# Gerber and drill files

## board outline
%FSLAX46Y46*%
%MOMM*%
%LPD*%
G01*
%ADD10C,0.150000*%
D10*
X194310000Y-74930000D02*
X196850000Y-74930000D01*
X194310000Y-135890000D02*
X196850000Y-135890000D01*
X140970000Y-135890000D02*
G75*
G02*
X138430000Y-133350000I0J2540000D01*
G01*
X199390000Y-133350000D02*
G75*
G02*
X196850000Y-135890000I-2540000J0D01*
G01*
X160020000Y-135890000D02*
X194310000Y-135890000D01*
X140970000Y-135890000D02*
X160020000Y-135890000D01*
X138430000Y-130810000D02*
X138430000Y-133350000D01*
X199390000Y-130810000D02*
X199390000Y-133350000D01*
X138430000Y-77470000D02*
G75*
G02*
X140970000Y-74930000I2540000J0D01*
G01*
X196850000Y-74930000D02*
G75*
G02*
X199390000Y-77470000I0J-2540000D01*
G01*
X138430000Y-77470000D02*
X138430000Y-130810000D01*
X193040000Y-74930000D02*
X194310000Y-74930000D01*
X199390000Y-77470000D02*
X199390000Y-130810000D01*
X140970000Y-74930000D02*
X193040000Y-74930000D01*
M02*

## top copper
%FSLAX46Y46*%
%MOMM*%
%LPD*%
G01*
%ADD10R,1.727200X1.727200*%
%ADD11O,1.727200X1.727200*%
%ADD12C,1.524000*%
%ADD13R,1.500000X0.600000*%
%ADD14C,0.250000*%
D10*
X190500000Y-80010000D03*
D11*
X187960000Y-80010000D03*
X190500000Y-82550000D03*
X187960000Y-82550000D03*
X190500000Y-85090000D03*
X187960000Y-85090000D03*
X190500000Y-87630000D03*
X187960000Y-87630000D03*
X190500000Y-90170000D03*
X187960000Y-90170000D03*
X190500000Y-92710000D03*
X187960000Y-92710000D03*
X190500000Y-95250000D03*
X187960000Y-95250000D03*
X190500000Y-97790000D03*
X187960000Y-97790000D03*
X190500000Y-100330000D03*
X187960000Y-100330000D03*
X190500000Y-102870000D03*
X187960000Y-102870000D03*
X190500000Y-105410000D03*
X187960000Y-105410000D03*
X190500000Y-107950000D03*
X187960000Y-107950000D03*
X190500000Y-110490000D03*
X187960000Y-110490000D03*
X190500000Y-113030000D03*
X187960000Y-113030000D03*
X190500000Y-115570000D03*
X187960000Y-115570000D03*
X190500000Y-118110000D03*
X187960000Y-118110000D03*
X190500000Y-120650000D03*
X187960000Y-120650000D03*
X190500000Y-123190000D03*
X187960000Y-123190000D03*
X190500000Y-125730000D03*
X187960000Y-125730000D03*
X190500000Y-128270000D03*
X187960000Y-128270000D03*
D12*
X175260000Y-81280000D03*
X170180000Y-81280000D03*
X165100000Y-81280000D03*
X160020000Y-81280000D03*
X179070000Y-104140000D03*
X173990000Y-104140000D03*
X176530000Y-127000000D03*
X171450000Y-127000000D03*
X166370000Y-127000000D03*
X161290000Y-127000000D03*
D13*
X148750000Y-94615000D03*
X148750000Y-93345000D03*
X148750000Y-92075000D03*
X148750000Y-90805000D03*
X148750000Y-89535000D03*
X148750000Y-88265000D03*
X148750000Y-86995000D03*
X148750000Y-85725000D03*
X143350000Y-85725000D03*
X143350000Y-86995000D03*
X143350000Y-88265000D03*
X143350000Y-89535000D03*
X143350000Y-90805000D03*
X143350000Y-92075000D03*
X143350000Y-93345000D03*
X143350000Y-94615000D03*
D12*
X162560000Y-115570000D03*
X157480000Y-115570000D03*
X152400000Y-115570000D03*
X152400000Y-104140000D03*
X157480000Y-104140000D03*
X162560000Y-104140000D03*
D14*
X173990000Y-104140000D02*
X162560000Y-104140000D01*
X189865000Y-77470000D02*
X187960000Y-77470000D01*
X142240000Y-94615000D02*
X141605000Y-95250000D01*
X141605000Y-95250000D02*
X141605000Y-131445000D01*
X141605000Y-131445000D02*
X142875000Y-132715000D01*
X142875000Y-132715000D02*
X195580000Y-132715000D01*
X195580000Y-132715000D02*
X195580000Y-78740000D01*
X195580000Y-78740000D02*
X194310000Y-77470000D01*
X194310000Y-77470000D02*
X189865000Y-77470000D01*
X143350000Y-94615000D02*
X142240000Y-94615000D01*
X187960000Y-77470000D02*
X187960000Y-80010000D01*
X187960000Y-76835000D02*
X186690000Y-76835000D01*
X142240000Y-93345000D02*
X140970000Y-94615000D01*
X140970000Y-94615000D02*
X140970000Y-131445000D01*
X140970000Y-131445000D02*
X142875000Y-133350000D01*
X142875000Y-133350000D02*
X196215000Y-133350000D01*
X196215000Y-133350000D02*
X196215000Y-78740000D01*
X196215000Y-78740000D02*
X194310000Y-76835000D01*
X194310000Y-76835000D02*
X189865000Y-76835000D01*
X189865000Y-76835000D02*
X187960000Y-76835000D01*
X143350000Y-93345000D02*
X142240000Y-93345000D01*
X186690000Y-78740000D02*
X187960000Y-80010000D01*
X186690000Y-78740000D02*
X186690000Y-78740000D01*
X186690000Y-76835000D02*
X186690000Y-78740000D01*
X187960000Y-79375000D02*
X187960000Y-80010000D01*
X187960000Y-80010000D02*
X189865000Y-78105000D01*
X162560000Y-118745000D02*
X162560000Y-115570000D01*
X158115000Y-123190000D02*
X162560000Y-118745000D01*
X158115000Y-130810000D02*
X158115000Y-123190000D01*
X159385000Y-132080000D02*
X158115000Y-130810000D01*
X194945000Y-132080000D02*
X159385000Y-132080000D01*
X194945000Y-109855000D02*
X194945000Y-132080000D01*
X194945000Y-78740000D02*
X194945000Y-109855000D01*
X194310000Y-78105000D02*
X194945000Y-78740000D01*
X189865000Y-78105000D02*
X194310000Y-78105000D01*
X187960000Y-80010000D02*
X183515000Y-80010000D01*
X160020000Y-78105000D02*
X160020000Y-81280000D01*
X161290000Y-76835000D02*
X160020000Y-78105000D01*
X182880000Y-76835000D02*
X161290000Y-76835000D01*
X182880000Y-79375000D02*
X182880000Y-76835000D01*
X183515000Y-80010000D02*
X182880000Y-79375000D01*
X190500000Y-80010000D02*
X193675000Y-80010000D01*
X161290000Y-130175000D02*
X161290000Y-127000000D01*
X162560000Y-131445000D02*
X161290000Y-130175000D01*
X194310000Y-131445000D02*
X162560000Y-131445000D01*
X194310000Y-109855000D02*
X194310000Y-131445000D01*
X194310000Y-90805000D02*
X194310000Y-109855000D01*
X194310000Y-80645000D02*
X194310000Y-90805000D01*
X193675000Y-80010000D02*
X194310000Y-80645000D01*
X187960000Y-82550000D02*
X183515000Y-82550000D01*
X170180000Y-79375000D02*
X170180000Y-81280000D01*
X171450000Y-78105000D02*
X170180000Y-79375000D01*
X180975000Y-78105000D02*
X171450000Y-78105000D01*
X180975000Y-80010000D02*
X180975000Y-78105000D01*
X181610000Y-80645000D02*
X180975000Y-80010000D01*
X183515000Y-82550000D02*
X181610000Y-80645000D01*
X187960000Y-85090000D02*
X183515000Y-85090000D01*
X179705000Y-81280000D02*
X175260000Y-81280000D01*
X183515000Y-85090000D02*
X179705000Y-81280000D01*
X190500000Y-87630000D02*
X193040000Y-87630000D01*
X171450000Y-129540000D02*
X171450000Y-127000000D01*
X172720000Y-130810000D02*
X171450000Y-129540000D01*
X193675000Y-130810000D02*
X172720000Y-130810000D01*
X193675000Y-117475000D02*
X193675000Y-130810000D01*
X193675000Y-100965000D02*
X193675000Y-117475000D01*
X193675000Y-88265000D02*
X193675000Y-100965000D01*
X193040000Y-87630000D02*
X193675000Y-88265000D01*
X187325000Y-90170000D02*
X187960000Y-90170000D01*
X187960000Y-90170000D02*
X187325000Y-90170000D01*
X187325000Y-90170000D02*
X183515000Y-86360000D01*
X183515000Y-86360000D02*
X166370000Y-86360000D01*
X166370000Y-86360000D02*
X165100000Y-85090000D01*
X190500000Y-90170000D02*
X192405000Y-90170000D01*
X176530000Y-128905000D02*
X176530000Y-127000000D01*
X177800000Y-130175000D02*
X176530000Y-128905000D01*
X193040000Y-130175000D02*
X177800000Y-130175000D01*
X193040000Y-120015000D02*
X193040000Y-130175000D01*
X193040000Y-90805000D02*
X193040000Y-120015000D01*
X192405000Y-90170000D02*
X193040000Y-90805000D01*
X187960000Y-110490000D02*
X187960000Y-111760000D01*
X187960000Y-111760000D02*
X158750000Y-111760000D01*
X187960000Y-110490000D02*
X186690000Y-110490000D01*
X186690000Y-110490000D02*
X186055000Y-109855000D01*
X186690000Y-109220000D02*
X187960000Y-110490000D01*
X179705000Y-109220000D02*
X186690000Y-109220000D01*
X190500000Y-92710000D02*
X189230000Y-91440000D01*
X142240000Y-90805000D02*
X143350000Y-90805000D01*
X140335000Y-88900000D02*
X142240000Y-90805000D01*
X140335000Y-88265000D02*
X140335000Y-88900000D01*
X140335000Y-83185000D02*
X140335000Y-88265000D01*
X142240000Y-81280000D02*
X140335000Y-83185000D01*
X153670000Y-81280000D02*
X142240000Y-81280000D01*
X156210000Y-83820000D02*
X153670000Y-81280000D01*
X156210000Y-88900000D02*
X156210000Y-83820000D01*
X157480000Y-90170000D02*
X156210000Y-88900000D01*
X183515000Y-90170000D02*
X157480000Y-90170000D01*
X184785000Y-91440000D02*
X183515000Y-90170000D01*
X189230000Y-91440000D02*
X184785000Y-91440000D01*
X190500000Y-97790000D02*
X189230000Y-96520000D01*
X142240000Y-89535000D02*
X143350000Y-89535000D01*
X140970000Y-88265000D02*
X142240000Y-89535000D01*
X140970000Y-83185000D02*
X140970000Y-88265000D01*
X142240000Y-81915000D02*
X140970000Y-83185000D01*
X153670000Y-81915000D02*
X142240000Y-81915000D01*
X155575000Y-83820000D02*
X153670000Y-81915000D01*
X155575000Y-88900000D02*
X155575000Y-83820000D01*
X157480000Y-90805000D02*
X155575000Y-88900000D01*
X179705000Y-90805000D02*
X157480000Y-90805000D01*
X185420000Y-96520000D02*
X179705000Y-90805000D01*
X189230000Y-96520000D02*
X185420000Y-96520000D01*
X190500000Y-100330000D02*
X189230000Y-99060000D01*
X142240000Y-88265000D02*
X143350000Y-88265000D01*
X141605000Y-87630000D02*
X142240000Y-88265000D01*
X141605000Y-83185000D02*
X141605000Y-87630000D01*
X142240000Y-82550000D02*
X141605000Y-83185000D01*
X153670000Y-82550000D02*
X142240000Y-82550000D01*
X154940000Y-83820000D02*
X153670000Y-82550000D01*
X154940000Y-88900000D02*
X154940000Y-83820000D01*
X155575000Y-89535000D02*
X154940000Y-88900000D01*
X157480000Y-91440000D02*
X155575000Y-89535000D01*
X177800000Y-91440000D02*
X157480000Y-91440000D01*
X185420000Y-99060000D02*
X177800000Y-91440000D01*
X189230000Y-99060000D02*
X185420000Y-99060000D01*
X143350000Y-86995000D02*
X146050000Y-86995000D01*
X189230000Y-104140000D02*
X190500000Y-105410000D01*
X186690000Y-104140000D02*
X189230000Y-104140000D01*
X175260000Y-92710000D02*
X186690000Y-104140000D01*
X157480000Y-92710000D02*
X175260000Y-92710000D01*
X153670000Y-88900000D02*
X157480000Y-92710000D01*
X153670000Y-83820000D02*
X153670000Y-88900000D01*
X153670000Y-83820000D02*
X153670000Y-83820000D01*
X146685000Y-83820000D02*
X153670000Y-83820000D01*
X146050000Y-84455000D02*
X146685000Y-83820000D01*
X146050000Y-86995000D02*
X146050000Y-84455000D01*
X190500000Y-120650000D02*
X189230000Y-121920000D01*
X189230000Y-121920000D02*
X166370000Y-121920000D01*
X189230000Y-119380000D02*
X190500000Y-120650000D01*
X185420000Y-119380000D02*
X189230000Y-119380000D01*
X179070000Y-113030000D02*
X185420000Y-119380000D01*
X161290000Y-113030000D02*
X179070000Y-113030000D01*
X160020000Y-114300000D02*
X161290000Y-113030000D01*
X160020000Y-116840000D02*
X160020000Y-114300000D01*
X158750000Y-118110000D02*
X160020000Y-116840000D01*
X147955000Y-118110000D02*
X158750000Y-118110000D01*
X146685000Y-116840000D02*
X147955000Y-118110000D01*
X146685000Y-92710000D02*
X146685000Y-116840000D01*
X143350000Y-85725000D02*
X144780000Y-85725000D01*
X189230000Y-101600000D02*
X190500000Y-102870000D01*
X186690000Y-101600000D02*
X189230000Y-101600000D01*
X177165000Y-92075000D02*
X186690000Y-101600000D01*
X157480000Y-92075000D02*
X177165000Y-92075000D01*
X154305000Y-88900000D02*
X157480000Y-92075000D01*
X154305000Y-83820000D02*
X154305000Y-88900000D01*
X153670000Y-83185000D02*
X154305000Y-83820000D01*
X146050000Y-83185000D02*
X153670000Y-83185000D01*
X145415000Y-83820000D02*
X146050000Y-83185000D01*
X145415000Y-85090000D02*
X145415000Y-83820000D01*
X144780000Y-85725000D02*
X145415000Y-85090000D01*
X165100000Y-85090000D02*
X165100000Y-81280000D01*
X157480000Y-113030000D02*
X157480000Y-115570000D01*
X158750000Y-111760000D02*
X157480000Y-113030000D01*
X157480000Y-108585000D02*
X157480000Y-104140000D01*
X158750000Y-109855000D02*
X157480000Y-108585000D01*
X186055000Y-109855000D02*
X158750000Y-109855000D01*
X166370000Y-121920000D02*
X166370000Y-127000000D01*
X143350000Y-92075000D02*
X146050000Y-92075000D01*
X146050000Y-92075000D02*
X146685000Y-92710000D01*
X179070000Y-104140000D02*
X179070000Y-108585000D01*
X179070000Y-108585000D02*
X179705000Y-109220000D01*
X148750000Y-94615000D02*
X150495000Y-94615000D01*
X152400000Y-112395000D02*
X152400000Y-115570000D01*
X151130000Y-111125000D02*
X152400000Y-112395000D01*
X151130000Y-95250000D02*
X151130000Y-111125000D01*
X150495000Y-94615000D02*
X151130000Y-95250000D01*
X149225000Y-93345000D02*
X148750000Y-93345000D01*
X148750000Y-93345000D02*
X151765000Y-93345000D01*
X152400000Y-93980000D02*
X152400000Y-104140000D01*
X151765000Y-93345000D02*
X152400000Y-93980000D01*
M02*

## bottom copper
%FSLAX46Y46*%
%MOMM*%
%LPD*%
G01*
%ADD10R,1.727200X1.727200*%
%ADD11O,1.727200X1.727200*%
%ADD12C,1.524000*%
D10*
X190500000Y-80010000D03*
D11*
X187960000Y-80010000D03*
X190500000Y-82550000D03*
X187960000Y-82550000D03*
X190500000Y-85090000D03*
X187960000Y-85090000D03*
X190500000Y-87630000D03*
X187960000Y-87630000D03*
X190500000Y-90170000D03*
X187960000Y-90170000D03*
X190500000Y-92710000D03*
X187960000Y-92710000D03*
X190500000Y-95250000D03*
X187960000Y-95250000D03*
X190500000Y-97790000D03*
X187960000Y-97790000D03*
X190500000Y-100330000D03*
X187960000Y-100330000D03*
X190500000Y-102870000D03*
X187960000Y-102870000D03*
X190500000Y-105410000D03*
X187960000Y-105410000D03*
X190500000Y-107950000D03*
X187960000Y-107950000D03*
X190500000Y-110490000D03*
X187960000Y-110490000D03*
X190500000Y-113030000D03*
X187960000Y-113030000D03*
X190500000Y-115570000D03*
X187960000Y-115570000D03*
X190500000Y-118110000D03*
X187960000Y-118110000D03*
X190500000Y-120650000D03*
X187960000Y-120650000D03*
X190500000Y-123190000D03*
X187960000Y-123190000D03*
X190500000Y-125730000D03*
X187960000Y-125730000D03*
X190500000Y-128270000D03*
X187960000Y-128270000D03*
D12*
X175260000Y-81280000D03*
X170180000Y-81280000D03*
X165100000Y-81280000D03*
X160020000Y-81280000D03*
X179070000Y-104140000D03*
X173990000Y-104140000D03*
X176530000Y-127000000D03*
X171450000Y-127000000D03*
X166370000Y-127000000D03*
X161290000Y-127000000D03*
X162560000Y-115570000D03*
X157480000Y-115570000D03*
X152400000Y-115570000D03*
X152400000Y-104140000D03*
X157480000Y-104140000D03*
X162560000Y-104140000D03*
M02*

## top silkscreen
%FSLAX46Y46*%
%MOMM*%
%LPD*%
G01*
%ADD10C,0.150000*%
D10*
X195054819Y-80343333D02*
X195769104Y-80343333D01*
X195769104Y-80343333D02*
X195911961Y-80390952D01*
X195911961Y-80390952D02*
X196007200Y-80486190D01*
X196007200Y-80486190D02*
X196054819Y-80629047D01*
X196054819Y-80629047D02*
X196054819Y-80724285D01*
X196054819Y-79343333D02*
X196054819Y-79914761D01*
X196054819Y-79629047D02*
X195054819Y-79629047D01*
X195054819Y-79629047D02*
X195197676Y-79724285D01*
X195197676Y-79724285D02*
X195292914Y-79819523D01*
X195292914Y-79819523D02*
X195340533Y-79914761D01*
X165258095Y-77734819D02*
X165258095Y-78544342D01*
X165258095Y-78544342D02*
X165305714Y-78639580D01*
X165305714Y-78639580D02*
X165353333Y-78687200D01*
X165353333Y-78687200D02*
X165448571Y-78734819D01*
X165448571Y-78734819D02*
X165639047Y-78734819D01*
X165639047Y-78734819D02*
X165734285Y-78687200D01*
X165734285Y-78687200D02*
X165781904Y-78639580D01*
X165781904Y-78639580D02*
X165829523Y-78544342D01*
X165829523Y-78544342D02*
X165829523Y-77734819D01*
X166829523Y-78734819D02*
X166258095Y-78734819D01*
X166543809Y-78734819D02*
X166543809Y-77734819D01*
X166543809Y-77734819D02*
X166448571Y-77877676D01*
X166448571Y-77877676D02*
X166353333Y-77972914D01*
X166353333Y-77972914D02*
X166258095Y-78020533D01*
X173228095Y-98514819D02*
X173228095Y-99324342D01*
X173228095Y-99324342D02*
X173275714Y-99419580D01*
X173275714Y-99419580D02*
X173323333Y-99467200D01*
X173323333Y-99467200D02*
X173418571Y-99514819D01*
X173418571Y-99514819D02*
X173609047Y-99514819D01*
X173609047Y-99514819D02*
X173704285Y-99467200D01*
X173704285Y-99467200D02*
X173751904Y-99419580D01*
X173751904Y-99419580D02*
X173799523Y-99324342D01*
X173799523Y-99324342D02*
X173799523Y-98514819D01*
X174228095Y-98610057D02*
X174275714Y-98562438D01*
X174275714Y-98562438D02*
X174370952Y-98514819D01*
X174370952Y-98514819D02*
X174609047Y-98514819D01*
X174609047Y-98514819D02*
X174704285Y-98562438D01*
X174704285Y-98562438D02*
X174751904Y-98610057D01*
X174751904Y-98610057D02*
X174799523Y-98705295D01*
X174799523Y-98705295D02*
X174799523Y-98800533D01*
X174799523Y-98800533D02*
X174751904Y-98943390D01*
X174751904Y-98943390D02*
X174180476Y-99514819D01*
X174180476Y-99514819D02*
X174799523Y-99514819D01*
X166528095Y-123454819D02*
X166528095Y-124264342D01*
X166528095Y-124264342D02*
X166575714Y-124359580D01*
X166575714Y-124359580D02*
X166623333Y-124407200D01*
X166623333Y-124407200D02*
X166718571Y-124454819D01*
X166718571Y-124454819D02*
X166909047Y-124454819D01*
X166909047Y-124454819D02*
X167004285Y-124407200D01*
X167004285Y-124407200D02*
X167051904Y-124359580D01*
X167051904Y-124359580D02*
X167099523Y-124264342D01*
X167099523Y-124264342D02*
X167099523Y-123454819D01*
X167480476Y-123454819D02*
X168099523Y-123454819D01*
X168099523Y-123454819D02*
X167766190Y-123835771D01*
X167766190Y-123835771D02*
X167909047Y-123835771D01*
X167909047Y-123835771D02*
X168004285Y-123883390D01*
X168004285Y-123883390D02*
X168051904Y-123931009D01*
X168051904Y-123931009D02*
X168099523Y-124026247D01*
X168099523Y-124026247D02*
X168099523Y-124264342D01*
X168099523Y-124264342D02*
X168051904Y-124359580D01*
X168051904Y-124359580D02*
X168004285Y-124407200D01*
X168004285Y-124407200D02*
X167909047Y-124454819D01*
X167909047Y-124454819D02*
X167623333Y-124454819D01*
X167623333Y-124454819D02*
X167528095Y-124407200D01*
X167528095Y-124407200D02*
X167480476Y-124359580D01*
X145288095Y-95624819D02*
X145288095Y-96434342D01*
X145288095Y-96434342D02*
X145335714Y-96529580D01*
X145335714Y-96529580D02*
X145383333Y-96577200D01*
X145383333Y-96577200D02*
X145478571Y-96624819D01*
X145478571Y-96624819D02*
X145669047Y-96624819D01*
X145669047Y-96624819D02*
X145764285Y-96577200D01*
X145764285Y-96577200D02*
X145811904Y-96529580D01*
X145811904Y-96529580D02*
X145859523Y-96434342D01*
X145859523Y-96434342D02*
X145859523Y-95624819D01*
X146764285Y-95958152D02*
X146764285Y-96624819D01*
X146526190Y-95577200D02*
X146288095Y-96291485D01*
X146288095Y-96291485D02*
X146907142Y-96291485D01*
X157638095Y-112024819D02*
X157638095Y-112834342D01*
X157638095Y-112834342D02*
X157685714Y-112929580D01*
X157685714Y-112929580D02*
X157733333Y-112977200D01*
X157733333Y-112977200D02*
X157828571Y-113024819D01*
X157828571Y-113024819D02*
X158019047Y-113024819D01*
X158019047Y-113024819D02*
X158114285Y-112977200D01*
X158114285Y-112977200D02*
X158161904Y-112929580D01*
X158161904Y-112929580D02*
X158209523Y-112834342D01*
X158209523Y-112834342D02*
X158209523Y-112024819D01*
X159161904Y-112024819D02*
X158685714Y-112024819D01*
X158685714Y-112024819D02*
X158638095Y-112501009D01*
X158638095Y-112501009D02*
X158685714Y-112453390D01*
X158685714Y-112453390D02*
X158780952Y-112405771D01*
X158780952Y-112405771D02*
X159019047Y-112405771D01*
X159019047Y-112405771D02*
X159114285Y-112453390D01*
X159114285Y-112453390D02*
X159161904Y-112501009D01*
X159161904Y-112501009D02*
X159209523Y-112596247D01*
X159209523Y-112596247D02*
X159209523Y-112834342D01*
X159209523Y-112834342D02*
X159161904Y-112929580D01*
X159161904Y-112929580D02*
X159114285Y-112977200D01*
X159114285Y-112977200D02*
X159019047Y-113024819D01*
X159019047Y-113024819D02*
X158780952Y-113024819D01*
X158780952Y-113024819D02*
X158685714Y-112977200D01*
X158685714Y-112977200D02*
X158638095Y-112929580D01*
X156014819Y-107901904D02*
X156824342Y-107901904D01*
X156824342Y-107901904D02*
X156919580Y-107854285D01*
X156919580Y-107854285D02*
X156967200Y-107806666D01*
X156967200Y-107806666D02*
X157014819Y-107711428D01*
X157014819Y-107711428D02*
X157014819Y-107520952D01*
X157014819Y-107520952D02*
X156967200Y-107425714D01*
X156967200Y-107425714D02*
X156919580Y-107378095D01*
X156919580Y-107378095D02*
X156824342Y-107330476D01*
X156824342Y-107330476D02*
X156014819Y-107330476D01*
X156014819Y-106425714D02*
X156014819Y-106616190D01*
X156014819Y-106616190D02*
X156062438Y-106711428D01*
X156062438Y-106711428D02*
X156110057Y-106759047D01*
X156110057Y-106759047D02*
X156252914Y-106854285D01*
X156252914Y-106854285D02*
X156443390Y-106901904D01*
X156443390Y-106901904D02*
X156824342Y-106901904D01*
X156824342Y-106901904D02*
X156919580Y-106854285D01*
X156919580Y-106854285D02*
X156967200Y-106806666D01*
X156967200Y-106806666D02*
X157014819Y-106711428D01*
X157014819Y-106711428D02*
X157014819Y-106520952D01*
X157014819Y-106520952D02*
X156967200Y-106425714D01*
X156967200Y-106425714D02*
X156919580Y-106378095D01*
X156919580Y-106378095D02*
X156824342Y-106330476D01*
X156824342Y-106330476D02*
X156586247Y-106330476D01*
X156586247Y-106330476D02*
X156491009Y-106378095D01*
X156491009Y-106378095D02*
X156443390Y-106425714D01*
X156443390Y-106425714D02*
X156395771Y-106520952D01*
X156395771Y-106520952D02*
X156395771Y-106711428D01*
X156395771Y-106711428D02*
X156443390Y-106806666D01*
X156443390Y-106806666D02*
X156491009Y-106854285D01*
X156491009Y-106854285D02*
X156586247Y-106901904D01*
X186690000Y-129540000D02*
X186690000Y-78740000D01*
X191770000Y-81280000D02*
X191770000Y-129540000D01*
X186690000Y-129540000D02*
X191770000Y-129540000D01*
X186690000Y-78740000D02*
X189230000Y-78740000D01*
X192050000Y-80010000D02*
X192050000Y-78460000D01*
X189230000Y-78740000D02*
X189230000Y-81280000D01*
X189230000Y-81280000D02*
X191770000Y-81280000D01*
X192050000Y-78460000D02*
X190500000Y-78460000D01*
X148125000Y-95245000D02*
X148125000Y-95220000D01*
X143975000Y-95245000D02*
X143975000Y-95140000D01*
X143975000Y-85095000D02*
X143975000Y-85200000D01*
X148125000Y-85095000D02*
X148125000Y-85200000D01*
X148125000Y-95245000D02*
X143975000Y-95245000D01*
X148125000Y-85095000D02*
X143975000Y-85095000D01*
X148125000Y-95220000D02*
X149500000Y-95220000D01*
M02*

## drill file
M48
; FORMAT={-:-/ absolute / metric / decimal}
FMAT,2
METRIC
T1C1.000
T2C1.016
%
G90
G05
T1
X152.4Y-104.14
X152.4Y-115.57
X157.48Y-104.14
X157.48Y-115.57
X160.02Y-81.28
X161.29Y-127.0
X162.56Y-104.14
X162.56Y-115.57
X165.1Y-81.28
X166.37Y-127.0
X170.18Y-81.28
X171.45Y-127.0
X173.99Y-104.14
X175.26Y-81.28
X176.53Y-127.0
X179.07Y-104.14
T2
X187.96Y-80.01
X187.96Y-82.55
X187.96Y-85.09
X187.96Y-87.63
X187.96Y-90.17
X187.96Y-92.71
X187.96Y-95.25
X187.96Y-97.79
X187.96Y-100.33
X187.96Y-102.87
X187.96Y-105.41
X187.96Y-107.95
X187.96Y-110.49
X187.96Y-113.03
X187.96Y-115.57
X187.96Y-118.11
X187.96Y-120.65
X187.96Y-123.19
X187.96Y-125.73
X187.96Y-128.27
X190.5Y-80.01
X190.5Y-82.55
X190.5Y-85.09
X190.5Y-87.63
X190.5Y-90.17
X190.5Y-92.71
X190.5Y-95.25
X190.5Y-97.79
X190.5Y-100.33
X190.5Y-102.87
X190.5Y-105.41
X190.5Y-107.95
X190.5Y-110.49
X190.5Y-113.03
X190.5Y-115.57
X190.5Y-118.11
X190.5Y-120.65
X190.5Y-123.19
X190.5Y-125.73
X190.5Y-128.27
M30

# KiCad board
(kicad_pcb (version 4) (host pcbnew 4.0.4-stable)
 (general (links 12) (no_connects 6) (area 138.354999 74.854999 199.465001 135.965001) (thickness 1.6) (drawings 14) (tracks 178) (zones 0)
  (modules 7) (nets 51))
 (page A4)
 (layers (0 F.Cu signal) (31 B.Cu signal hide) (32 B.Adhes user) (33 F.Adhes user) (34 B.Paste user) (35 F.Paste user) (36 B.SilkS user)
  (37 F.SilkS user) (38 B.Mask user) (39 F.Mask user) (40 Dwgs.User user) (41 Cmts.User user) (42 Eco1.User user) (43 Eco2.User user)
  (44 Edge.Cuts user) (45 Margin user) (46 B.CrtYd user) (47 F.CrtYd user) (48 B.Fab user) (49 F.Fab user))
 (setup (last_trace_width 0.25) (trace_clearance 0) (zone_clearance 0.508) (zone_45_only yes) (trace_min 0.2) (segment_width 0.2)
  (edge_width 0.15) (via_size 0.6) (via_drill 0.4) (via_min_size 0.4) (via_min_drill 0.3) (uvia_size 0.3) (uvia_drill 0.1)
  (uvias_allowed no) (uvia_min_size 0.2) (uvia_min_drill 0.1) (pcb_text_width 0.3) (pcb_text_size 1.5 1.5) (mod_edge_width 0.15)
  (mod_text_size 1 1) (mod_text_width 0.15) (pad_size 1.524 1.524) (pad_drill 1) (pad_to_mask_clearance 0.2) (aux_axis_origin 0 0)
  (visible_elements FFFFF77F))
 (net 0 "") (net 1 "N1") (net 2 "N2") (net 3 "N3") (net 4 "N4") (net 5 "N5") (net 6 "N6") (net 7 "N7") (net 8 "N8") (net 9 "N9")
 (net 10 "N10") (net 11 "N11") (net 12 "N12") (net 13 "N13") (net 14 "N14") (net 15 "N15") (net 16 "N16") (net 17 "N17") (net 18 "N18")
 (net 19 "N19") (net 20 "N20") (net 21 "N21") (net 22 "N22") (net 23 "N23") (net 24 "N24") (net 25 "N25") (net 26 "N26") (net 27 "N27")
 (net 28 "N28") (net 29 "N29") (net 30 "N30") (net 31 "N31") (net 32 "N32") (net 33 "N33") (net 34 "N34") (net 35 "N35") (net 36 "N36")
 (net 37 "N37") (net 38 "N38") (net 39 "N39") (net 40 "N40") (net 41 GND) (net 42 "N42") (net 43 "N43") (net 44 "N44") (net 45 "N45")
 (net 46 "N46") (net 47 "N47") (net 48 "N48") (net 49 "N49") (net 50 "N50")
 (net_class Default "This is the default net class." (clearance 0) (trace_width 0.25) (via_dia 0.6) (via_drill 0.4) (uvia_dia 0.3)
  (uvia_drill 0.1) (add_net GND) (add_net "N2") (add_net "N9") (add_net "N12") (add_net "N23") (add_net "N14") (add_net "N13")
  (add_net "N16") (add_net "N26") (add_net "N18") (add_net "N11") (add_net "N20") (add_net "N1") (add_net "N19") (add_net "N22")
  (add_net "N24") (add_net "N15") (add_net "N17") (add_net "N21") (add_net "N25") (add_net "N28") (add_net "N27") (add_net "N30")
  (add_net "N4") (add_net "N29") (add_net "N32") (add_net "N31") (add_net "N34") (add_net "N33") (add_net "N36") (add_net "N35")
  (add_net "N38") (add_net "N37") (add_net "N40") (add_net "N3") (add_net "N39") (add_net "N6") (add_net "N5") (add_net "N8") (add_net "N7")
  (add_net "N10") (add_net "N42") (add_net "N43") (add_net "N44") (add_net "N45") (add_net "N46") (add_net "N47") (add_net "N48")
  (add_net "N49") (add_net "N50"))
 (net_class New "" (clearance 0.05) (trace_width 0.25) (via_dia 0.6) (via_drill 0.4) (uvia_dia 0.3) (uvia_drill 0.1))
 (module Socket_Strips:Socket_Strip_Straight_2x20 (layer F.Cu) (at 190.5 80.01 270)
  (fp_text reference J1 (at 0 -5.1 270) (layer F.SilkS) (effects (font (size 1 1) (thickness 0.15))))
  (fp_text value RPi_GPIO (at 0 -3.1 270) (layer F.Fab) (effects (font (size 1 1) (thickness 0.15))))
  (fp_line (start 49.53 3.81) (end -1.27 3.81) (layer F.SilkS) (width 0.15))
  (fp_line (start 1.27 -1.27) (end 49.53 -1.27) (layer F.SilkS) (width 0.15))
  (fp_line (start 49.53 3.81) (end 49.53 -1.27) (layer F.SilkS) (width 0.15))
  (fp_line (start -1.27 3.81) (end -1.27 1.27) (layer F.SilkS) (width 0.15))
  (fp_line (start 0 -1.55) (end -1.55 -1.55) (layer F.SilkS) (width 0.15))
  (fp_line (start -1.27 1.27) (end 1.27 1.27) (layer F.SilkS) (width 0.15))
  (fp_line (start 1.27 1.27) (end 1.27 -1.27) (layer F.SilkS) (width 0.15))
  (fp_line (start -1.55 -1.55) (end -1.55 0) (layer F.SilkS) (width 0.15))
  (pad 2 thru_hole rect (at 0 0 270) (size 1.7272 1.7272) (drill 1.016) (layers *.Cu *.Mask) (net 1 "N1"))
  (pad 1 thru_hole oval (at 0 2.54 270) (size 1.7272 1.7272) (drill 1.016) (layers *.Cu *.Mask) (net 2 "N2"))
  (pad 4 thru_hole oval (at 2.54 0 270) (size 1.7272 1.7272) (drill 1.016) (layers *.Cu *.Mask) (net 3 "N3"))
  (pad 3 thru_hole oval (at 2.54 2.54 270) (size 1.7272 1.7272) (drill 1.016) (layers *.Cu *.Mask) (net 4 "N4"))
  (pad 6 thru_hole oval (at 5.08 0 270) (size 1.7272 1.7272) (drill 1.016) (layers *.Cu *.Mask) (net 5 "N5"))
  (pad 5 thru_hole oval (at 5.08 2.54 270) (size 1.7272 1.7272) (drill 1.016) (layers *.Cu *.Mask) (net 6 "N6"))
  (pad 8 thru_hole oval (at 7.62 0 270) (size 1.7272 1.7272) (drill 1.016) (layers *.Cu *.Mask) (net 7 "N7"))
  (pad 7 thru_hole oval (at 7.62 2.54 270) (size 1.7272 1.7272) (drill 1.016) (layers *.Cu *.Mask) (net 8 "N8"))
  (pad 10 thru_hole oval (at 10.16 0 270) (size 1.7272 1.7272) (drill 1.016) (layers *.Cu *.Mask) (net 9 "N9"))
  (pad 9 thru_hole oval (at 10.16 2.54 270) (size 1.7272 1.7272) (drill 1.016) (layers *.Cu *.Mask) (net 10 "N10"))
  (pad 18 thru_hole oval (at 12.7 0 270) (size 1.7272 1.7272) (drill 1.016) (layers *.Cu *.Mask) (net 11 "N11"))
  (pad 11 thru_hole oval (at 12.7 2.54 270) (size 1.7272 1.7272) (drill 1.016) (layers *.Cu *.Mask) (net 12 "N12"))
  (pad 14 thru_hole oval (at 15.24 0 270) (size 1.7272 1.7272) (drill 1.016) (layers *.Cu *.Mask) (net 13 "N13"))
  (pad 13 thru_hole oval (at 15.24 2.54 270) (size 1.7272 1.7272) (drill 1.016) (layers *.Cu *.Mask) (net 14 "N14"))
  (pad 23 thru_hole oval (at 17.78 0 270) (size 1.7272 1.7272) (drill 1.016) (layers *.Cu *.Mask) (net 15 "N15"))
  (pad 15 thru_hole oval (at 17.78 2.54 270) (size 1.7272 1.7272) (drill 1.016) (layers *.Cu *.Mask) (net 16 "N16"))
  (pad 24 thru_hole oval (at 20.32 0 270) (size 1.7272 1.7272) (drill 1.016) (layers *.Cu *.Mask) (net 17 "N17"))
  (pad 17 thru_hole oval (at 20.32 2.54 270) (size 1.7272 1.7272) (drill 1.016) (layers *.Cu *.Mask) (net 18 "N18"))
  (pad 20 thru_hole oval (at 22.86 0 270) (size 1.7272 1.7272) (drill 1.016) (layers *.Cu *.Mask) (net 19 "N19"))
  (pad 19 thru_hole oval (at 22.86 2.54 270) (size 1.7272 1.7272) (drill 1.016) (layers *.Cu *.Mask) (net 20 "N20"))
  (pad 25 thru_hole oval (at 25.4 0 270) (size 1.7272 1.7272) (drill 1.016) (layers *.Cu *.Mask) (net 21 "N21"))
  (pad 21 thru_hole oval (at 25.4 2.54 270) (size 1.7272 1.7272) (drill 1.016) (layers *.Cu *.Mask) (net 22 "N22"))
  (pad 12 thru_hole oval (at 27.94 0 270) (size 1.7272 1.7272) (drill 1.016) (layers *.Cu *.Mask) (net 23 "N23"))
  (pad 22 thru_hole oval (at 27.94 2.54 270) (size 1.7272 1.7272) (drill 1.016) (layers *.Cu *.Mask) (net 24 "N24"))
  (pad 26 thru_hole oval (at 30.48 0 270) (size 1.7272 1.7272) (drill 1.016) (layers *.Cu *.Mask) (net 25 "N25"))
  (pad 16 thru_hole oval (at 30.48 2.54 270) (size 1.7272 1.7272) (drill 1.016) (layers *.Cu *.Mask) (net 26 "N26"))
  (pad 28 thru_hole oval (at 33.02 0 270) (size 1.7272 1.7272) (drill 1.016) (layers *.Cu *.Mask) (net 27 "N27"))
  (pad 27 thru_hole oval (at 33.02 2.54 270) (size 1.7272 1.7272) (drill 1.016) (layers *.Cu *.Mask) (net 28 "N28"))
  (pad 30 thru_hole oval (at 35.56 0 270) (size 1.7272 1.7272) (drill 1.016) (layers *.Cu *.Mask) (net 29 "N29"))
  (pad 29 thru_hole oval (at 35.56 2.54 270) (size 1.7272 1.7272) (drill 1.016) (layers *.Cu *.Mask) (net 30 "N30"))
  (pad 32 thru_hole oval (at 38.1 0 270) (size 1.7272 1.7272) (drill 1.016) (layers *.Cu *.Mask) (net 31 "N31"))
  (pad 31 thru_hole oval (at 38.1 2.54 270) (size 1.7272 1.7272) (drill 1.016) (layers *.Cu *.Mask) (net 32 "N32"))
  (pad 34 thru_hole oval (at 40.64 0 270) (size 1.7272 1.7272) (drill 1.016) (layers *.Cu *.Mask) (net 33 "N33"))
  (pad 33 thru_hole oval (at 40.64 2.54 270) (size 1.7272 1.7272) (drill 1.016) (layers *.Cu *.Mask) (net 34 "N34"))
  (pad 36 thru_hole oval (at 43.18 0 270) (size 1.7272 1.7272) (drill 1.016) (layers *.Cu *.Mask) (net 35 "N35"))
  (pad 35 thru_hole oval (at 43.18 2.54 270) (size 1.7272 1.7272) (drill 1.016) (layers *.Cu *.Mask) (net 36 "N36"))
  (pad 38 thru_hole oval (at 45.72 0 270) (size 1.7272 1.7272) (drill 1.016) (layers *.Cu *.Mask) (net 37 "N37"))
  (pad 37 thru_hole oval (at 45.72 2.54 270) (size 1.7272 1.7272) (drill 1.016) (layers *.Cu *.Mask) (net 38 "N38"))
  (pad 40 thru_hole oval (at 48.26 0 270) (size 1.7272 1.7272) (drill 1.016) (layers *.Cu *.Mask) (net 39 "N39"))
  (pad 39 thru_hole oval (at 48.26 2.54 270) (size 1.7272 1.7272) (drill 1.016) (layers *.Cu *.Mask) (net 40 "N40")))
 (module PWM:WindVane (layer F.Cu) (at 160.02 81.28)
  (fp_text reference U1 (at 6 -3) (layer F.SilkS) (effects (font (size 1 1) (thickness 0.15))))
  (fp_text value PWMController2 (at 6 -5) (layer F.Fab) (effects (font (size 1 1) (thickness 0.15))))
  (pad 4 thru_hole circle (at 15.24 0) (size 1.524 1.524) (drill 1) (layers *.Cu *.Mask))
  (pad 3 thru_hole circle (at 10.16 0) (size 1.524 1.524) (drill 1) (layers *.Cu *.Mask))
  (pad 2 thru_hole circle (at 5.08 0) (size 1.524 1.524) (drill 1) (layers *.Cu *.Mask) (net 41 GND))
  (pad 1 thru_hole circle (at 0 0) (size 1.524 1.524) (drill 1) (layers *.Cu *.Mask)))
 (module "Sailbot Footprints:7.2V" (layer F.Cu) (at 173.99 104.14)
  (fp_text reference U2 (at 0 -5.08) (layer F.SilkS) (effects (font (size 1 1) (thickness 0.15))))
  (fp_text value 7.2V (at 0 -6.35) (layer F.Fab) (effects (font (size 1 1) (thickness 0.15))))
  (pad 2 thru_hole circle (at 5.08 0) (size 1.524 1.524) (drill 1) (layers *.Cu *.Mask) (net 41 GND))
  (pad 1 thru_hole circle (at 0 0) (size 1.524 1.524) (drill 1) (layers *.Cu *.Mask) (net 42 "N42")))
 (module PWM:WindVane (layer F.Cu) (at 161.29 127)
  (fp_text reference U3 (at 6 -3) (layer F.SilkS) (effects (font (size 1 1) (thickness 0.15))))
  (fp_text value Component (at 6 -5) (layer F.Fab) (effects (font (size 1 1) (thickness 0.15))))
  (pad 4 thru_hole circle (at 15.24 0) (size 1.524 1.524) (drill 1) (layers *.Cu *.Mask))
  (pad 3 thru_hole circle (at 10.16 0) (size 1.524 1.524) (drill 1) (layers *.Cu *.Mask))
  (pad 2 thru_hole circle (at 5.08 0) (size 1.524 1.524) (drill 1) (layers *.Cu *.Mask) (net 41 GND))
  (pad 1 thru_hole circle (at 0 0) (size 1.524 1.524) (drill 1) (layers *.Cu *.Mask)))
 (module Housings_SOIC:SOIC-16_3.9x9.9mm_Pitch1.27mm (layer F.Cu) (at 146.05 90.17 180)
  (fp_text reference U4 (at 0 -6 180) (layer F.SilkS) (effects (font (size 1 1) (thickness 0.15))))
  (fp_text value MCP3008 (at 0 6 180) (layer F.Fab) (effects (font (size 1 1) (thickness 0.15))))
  (fp_line (start -2.075 -5.075) (end -2.075 -5.05) (layer F.SilkS) (width 0.15))
  (fp_line (start 2.075 -5.075) (end 2.075 -4.97) (layer F.SilkS) (width 0.15))
  (fp_line (start 2.075 5.075) (end 2.075 4.97) (layer F.SilkS) (width 0.15))
  (fp_line (start -2.075 5.075) (end -2.075 4.97) (layer F.SilkS) (width 0.15))
  (fp_line (start -2.075 -5.075) (end 2.075 -5.075) (layer F.SilkS) (width 0.15))
  (fp_line (start -2.075 5.075) (end 2.075 5.075) (layer F.SilkS) (width 0.15))
  (fp_line (start -2.075 -5.05) (end -3.45 -5.05) (layer F.SilkS) (width 0.15))
  (pad 1 smd rect (at -2.7 -4.445 180) (size 1.5 0.6) (layers F.Cu F.Paste F.Mask) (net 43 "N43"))
  (pad 2 smd rect (at -2.7 -3.175 180) (size 1.5 0.6) (layers F.Cu F.Paste F.Mask) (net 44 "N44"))
  (pad 3 smd rect (at -2.7 -1.905 180) (size 1.5 0.6) (layers F.Cu F.Paste F.Mask) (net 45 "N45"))
  (pad 4 smd rect (at -2.7 -0.635 180) (size 1.5 0.6) (layers F.Cu F.Paste F.Mask) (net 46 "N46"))
  (pad 5 smd rect (at -2.7 0.635 180) (size 1.5 0.6) (layers F.Cu F.Paste F.Mask) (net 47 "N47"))
  (pad 6 smd rect (at -2.7 1.905 180) (size 1.5 0.6) (layers F.Cu F.Paste F.Mask) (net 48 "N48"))
  (pad 7 smd rect (at -2.7 3.175 180) (size 1.5 0.6) (layers F.Cu F.Paste F.Mask) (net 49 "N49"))
  (pad 8 smd rect (at -2.7 4.445 180) (size 1.5 0.6) (layers F.Cu F.Paste F.Mask) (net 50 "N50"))
  (pad 9 smd rect (at 2.7 4.445 180) (size 1.5 0.6) (layers F.Cu F.Paste F.Mask) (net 41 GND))
  (pad 10 smd rect (at 2.7 3.175 180) (size 1.5 0.6) (layers F.Cu F.Paste F.Mask) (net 21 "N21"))
  (pad 11 smd rect (at 2.7 1.905 180) (size 1.5 0.6) (layers F.Cu F.Paste F.Mask) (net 17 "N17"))
  (pad 12 smd rect (at 2.7 0.635 180) (size 1.5 0.6) (layers F.Cu F.Paste F.Mask) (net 15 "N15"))
  (pad 13 smd rect (at 2.7 -0.635 180) (size 1.5 0.6) (layers F.Cu F.Paste F.Mask) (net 11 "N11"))
  (pad 14 smd rect (at 2.7 -1.905 180) (size 1.5 0.6) (layers F.Cu F.Paste F.Mask) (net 41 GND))
  (pad 15 smd rect (at 2.7 -3.175 180) (size 1.5 0.6) (layers F.Cu F.Paste F.Mask) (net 2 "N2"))
  (pad 16 smd rect (at 2.7 -4.445 180) (size 1.5 0.6) (layers F.Cu F.Paste F.Mask) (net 2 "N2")))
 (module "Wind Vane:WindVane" (layer F.Cu) (at 152.4 115.57)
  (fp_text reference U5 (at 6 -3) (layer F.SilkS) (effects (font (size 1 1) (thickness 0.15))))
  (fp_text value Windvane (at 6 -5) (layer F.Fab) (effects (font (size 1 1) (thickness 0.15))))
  (pad 3 thru_hole circle (at 10.16 0) (size 1.524 1.524) (drill 1) (layers *.Cu *.Mask))
  (pad 2 thru_hole circle (at 5.08 0) (size 1.524 1.524) (drill 1) (layers *.Cu *.Mask) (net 41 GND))
  (pad 1 thru_hole circle (at 0 0) (size 1.524 1.524) (drill 1) (layers *.Cu *.Mask)))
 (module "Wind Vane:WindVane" (layer F.Cu) (at 162.56 104.14 180)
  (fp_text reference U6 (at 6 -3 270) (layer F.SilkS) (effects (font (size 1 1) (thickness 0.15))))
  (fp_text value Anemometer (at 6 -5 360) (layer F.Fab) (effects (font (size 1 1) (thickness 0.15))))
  (pad 3 thru_hole circle (at 10.16 0 180) (size 1.524 1.524) (drill 1) (layers *.Cu *.Mask))
  (pad 2 thru_hole circle (at 5.08 0 180) (size 1.524 1.524) (drill 1) (layers *.Cu *.Mask) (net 41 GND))
  (pad 1 thru_hole circle (at 0 0 180) (size 1.524 1.524) (drill 1) (layers *.Cu *.Mask)))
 (gr_line (start 194.31 74.93) (end 196.85 74.93) (angle 90) (layer Edge.Cuts) (width 0.15))
 (gr_line (start 194.31 135.89) (end 196.85 135.89) (angle 90) (layer Edge.Cuts) (width 0.15))
 (gr_arc (start 140.97 133.35) (end 140.97 135.89) (angle 90) (layer Edge.Cuts) (width 0.15))
 (gr_arc (start 196.85 133.35) (end 199.39 133.35) (angle 90) (layer Edge.Cuts) (width 0.15))
 (gr_line (start 160.02 135.89) (end 194.31 135.89) (angle 90) (layer Edge.Cuts) (width 0.15))
 (gr_line (start 140.97 135.89) (end 160.02 135.89) (angle 90) (layer Edge.Cuts) (width 0.15))
 (gr_line (start 138.43 130.81) (end 138.43 133.35) (angle 90) (layer Edge.Cuts) (width 0.15))
 (gr_line (start 199.39 130.81) (end 199.39 133.35) (angle 90) (layer Edge.Cuts) (width 0.15))
 (gr_arc (start 140.97 77.47) (end 138.43 77.47) (angle 90) (layer Edge.Cuts) (width 0.15))
 (gr_arc (start 196.85 77.47) (end 196.85 74.93) (angle 90) (layer Edge.Cuts) (width 0.15))
 (gr_line (start 138.43 77.47) (end 138.43 130.81) (angle 90) (layer Edge.Cuts) (width 0.15))
 (gr_line (start 193.04 74.93) (end 194.31 74.93) (angle 90) (layer Edge.Cuts) (width 0.15))
 (gr_line (start 199.39 77.47) (end 199.39 130.81) (angle 90) (layer Edge.Cuts) (width 0.15))
 (gr_line (start 140.97 74.93) (end 193.04 74.93) (angle 90) (layer Edge.Cuts) (width 0.15))
 (segment (start 173.99 104.14) (end 162.56 104.14) (width 0.25) (layer F.Cu) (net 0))
 (segment (start 189.865 77.47) (end 187.96 77.47) (width 0.25) (layer F.Cu) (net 2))
 (segment (start 142.24 94.615) (end 141.605 95.25) (width 0.25) (layer F.Cu) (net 2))
 (segment (start 141.605 95.25) (end 141.605 131.445) (width 0.25) (layer F.Cu) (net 2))
 (segment (start 141.605 131.445) (end 142.875 132.715) (width 0.25) (layer F.Cu) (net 2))
 (segment (start 142.875 132.715) (end 195.58 132.715) (width 0.25) (layer F.Cu) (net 2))
 (segment (start 195.58 132.715) (end 195.58 78.74) (width 0.25) (layer F.Cu) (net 2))
 (segment (start 195.58 78.74) (end 194.31 77.47) (width 0.25) (layer F.Cu) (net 2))
 (segment (start 194.31 77.47) (end 189.865 77.47) (width 0.25) (layer F.Cu) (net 2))
 (segment (start 143.35 94.615) (end 142.24 94.615) (width 0.25) (layer F.Cu) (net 2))
 (segment (start 187.96 77.47) (end 187.96 80.01) (width 0.25) (layer F.Cu) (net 2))
 (segment (start 187.96 76.835) (end 186.69 76.835) (width 0.25) (layer F.Cu) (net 2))
 (segment (start 142.24 93.345) (end 140.97 94.615) (width 0.25) (layer F.Cu) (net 2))
 (segment (start 140.97 94.615) (end 140.97 131.445) (width 0.25) (layer F.Cu) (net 2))
 (segment (start 140.97 131.445) (end 142.875 133.35) (width 0.25) (layer F.Cu) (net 2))
 (segment (start 142.875 133.35) (end 196.215 133.35) (width 0.25) (layer F.Cu) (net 2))
 (segment (start 196.215 133.35) (end 196.215 78.74) (width 0.25) (layer F.Cu) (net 2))
 (segment (start 196.215 78.74) (end 194.31 76.835) (width 0.25) (layer F.Cu) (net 2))
 (segment (start 194.31 76.835) (end 189.865 76.835) (width 0.25) (layer F.Cu) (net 2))
 (segment (start 189.865 76.835) (end 187.96 76.835) (width 0.25) (layer F.Cu) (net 2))
 (segment (start 143.35 93.345) (end 142.24 93.345) (width 0.25) (layer F.Cu) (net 2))
 (segment (start 186.69 78.74) (end 187.96 80.01) (width 0.25) (layer F.Cu) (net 2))
 (segment (start 186.69 78.74) (end 186.69 78.74) (width 0.25) (layer F.Cu) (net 2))
 (segment (start 186.69 76.835) (end 186.69 78.74) (width 0.25) (layer F.Cu) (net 2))
 (segment (start 187.96 79.375) (end 187.96 80.01) (width 0.25) (layer F.Cu) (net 2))
 (segment (start 187.96 80.01) (end 189.865 78.105) (width 0.25) (layer F.Cu) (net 2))
 (segment (start 162.56 118.745) (end 162.56 115.57) (width 0.25) (layer F.Cu) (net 2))
 (segment (start 158.115 123.19) (end 162.56 118.745) (width 0.25) (layer F.Cu) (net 2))
 (segment (start 158.115 130.81) (end 158.115 123.19) (width 0.25) (layer F.Cu) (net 2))
 (segment (start 159.385 132.08) (end 158.115 130.81) (width 0.25) (layer F.Cu) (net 2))
 (segment (start 194.945 132.08) (end 159.385 132.08) (width 0.25) (layer F.Cu) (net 2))
 (segment (start 194.945 109.855) (end 194.945 132.08) (width 0.25) (layer F.Cu) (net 2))
 (segment (start 194.945 78.74) (end 194.945 109.855) (width 0.25) (layer F.Cu) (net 2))
 (segment (start 194.31 78.105) (end 194.945 78.74) (width 0.25) (layer F.Cu) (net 2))
 (segment (start 189.865 78.105) (end 194.31 78.105) (width 0.25) (layer F.Cu) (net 2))
 (segment (start 187.96 80.01) (end 183.515 80.01) (width 0.25) (layer F.Cu) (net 2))
 (segment (start 160.02 78.105) (end 160.02 81.28) (width 0.25) (layer F.Cu) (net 2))
 (segment (start 161.29 76.835) (end 160.02 78.105) (width 0.25) (layer F.Cu) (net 2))
 (segment (start 182.88 76.835) (end 161.29 76.835) (width 0.25) (layer F.Cu) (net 2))
 (segment (start 182.88 79.375) (end 182.88 76.835) (width 0.25) (layer F.Cu) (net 2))
 (segment (start 183.515 80.01) (end 182.88 79.375) (width 0.25) (layer F.Cu) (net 2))
 (segment (start 190.5 80.01) (end 193.675 80.01) (width 0.25) (layer F.Cu) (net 1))
 (segment (start 161.29 130.175) (end 161.29 127) (width 0.25) (layer F.Cu) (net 1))
 (segment (start 162.56 131.445) (end 161.29 130.175) (width 0.25) (layer F.Cu) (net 1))
 (segment (start 194.31 131.445) (end 162.56 131.445) (width 0.25) (layer F.Cu) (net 1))
 (segment (start 194.31 109.855) (end 194.31 131.445) (width 0.25) (layer F.Cu) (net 1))
 (segment (start 194.31 90.805) (end 194.31 109.855) (width 0.25) (layer F.Cu) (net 1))
 (segment (start 194.31 80.645) (end 194.31 90.805) (width 0.25) (layer F.Cu) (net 1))
 (segment (start 193.675 80.01) (end 194.31 80.645) (width 0.25) (layer F.Cu) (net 1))
 (segment (start 187.96 82.55) (end 183.515 82.55) (width 0.25) (layer F.Cu) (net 4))
 (segment (start 170.18 79.375) (end 170.18 81.28) (width 0.25) (layer F.Cu) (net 4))
 (segment (start 171.45 78.105) (end 170.18 79.375) (width 0.25) (layer F.Cu) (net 4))
 (segment (start 180.975 78.105) (end 171.45 78.105) (width 0.25) (layer F.Cu) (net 4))
 (segment (start 180.975 80.01) (end 180.975 78.105) (width 0.25) (layer F.Cu) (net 4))
 (segment (start 181.61 80.645) (end 180.975 80.01) (width 0.25) (layer F.Cu) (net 4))
 (segment (start 183.515 82.55) (end 181.61 80.645) (width 0.25) (layer F.Cu) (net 4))
 (segment (start 187.96 85.09) (end 183.515 85.09) (width 0.25) (layer F.Cu) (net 6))
 (segment (start 179.705 81.28) (end 175.26 81.28) (width 0.25) (layer F.Cu) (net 6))
 (segment (start 183.515 85.09) (end 179.705 81.28) (width 0.25) (layer F.Cu) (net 6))
 (segment (start 190.5 87.63) (end 193.04 87.63) (width 0.25) (layer F.Cu) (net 7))
 (segment (start 171.45 129.54) (end 171.45 127) (width 0.25) (layer F.Cu) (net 7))
 (segment (start 172.72 130.81) (end 171.45 129.54) (width 0.25) (layer F.Cu) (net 7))
 (segment (start 193.675 130.81) (end 172.72 130.81) (width 0.25) (layer F.Cu) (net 7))
 (segment (start 193.675 117.475) (end 193.675 130.81) (width 0.25) (layer F.Cu) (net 7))
 (segment (start 193.675 100.965) (end 193.675 117.475) (width 0.25) (layer F.Cu) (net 7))
 (segment (start 193.675 88.265) (end 193.675 100.965) (width 0.25) (layer F.Cu) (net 7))
 (segment (start 193.04 87.63) (end 193.675 88.265) (width 0.25) (layer F.Cu) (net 7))
 (segment (start 187.325 90.17) (end 187.96 90.17) (width 0.25) (layer F.Cu) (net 10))
 (segment (start 187.96 90.17) (end 187.325 90.17) (width 0.25) (layer F.Cu) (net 10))
 (segment (start 187.325 90.17) (end 183.515 86.36) (width 0.25) (layer F.Cu) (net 10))
 (segment (start 183.515 86.36) (end 166.37 86.36) (width 0.25) (layer F.Cu) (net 10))
 (segment (start 166.37 86.36) (end 165.1 85.09) (width 0.25) (layer F.Cu) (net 10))
 (segment (start 190.5 90.17) (end 192.405 90.17) (width 0.25) (layer F.Cu) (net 9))
 (segment (start 176.53 128.905) (end 176.53 127) (width 0.25) (layer F.Cu) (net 9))
 (segment (start 177.8 130.175) (end 176.53 128.905) (width 0.25) (layer F.Cu) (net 9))
 (segment (start 193.04 130.175) (end 177.8 130.175) (width 0.25) (layer F.Cu) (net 9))
 (segment (start 193.04 120.015) (end 193.04 130.175) (width 0.25) (layer F.Cu) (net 9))
 (segment (start 193.04 90.805) (end 193.04 120.015) (width 0.25) (layer F.Cu) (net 9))
 (segment (start 192.405 90.17) (end 193.04 90.805) (width 0.25) (layer F.Cu) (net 9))
 (segment (start 187.96 110.49) (end 187.96 111.76) (width 0.25) (layer F.Cu) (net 26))
 (segment (start 187.96 111.76) (end 158.75 111.76) (width 0.25) (layer F.Cu) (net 26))
 (segment (start 187.96 110.49) (end 186.69 110.49) (width 0.25) (layer F.Cu) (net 26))
 (segment (start 186.69 110.49) (end 186.055 109.855) (width 0.25) (layer F.Cu) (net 26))
 (segment (start 186.69 109.22) (end 187.96 110.49) (width 0.25) (layer F.Cu) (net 26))
 (segment (start 179.705 109.22) (end 186.69 109.22) (width 0.25) (layer F.Cu) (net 26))
 (segment (start 190.5 92.71) (end 189.23 91.44) (width 0.25) (layer F.Cu) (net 11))
 (segment (start 142.24 90.805) (end 143.35 90.805) (width 0.25) (layer F.Cu) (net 11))
 (segment (start 140.335 88.9) (end 142.24 90.805) (width 0.25) (layer F.Cu) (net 11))
 (segment (start 140.335 88.265) (end 140.335 88.9) (width 0.25) (layer F.Cu) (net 11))
 (segment (start 140.335 83.185) (end 140.335 88.265) (width 0.25) (layer F.Cu) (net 11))
 (segment (start 142.24 81.28) (end 140.335 83.185) (width 0.25) (layer F.Cu) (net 11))
 (segment (start 153.67 81.28) (end 142.24 81.28) (width 0.25) (layer F.Cu) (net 11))
 (segment (start 156.21 83.82) (end 153.67 81.28) (width 0.25) (layer F.Cu) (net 11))
 (segment (start 156.21 88.9) (end 156.21 83.82) (width 0.25) (layer F.Cu) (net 11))
 (segment (start 157.48 90.17) (end 156.21 88.9) (width 0.25) (layer F.Cu) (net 11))
 (segment (start 183.515 90.17) (end 157.48 90.17) (width 0.25) (layer F.Cu) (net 11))
 (segment (start 184.785 91.44) (end 183.515 90.17) (width 0.25) (layer F.Cu) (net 11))
 (segment (start 189.23 91.44) (end 184.785 91.44) (width 0.25) (layer F.Cu) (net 11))
 (segment (start 190.5 97.79) (end 189.23 96.52) (width 0.25) (layer F.Cu) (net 15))
 (segment (start 142.24 89.535) (end 143.35 89.535) (width 0.25) (layer F.Cu) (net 15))
 (segment (start 140.97 88.265) (end 142.24 89.535) (width 0.25) (layer F.Cu) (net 15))
 (segment (start 140.97 83.185) (end 140.97 88.265) (width 0.25) (layer F.Cu) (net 15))
 (segment (start 142.24 81.915) (end 140.97 83.185) (width 0.25) (layer F.Cu) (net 15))
 (segment (start 153.67 81.915) (end 142.24 81.915) (width 0.25) (layer F.Cu) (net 15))
 (segment (start 155.575 83.82) (end 153.67 81.915) (width 0.25) (layer F.Cu) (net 15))
 (segment (start 155.575 88.9) (end 155.575 83.82) (width 0.25) (layer F.Cu) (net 15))
 (segment (start 157.48 90.805) (end 155.575 88.9) (width 0.25) (layer F.Cu) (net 15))
 (segment (start 179.705 90.805) (end 157.48 90.805) (width 0.25) (layer F.Cu) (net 15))
 (segment (start 185.42 96.52) (end 179.705 90.805) (width 0.25) (layer F.Cu) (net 15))
 (segment (start 189.23 96.52) (end 185.42 96.52) (width 0.25) (layer F.Cu) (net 15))
 (segment (start 190.5 100.33) (end 189.23 99.06) (width 0.25) (layer F.Cu) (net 17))
 (segment (start 142.24 88.265) (end 143.35 88.265) (width 0.25) (layer F.Cu) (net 17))
 (segment (start 141.605 87.63) (end 142.24 88.265) (width 0.25) (layer F.Cu) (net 17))
 (segment (start 141.605 83.185) (end 141.605 87.63) (width 0.25) (layer F.Cu) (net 17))
 (segment (start 142.24 82.55) (end 141.605 83.185) (width 0.25) (layer F.Cu) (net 17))
 (segment (start 153.67 82.55) (end 142.24 82.55) (width 0.25) (layer F.Cu) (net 17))
 (segment (start 154.94 83.82) (end 153.67 82.55) (width 0.25) (layer F.Cu) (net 17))
 (segment (start 154.94 88.9) (end 154.94 83.82) (width 0.25) (layer F.Cu) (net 17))
 (segment (start 155.575 89.535) (end 154.94 88.9) (width 0.25) (layer F.Cu) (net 17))
 (segment (start 157.48 91.44) (end 155.575 89.535) (width 0.25) (layer F.Cu) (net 17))
 (segment (start 177.8 91.44) (end 157.48 91.44) (width 0.25) (layer F.Cu) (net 17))
 (segment (start 185.42 99.06) (end 177.8 91.44) (width 0.25) (layer F.Cu) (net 17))
 (segment (start 189.23 99.06) (end 185.42 99.06) (width 0.25) (layer F.Cu) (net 17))
 (segment (start 143.35 86.995) (end 146.05 86.995) (width 0.25) (layer F.Cu) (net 21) (status 400000))
 (segment (start 189.23 104.14) (end 190.5 105.41) (width 0.25) (layer F.Cu) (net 21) (status 800000))
 (segment (start 186.69 104.14) (end 189.23 104.14) (width 0.25) (layer F.Cu) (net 21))
 (segment (start 175.26 92.71) (end 186.69 104.14) (width 0.25) (layer F.Cu) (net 21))
 (segment (start 157.48 92.71) (end 175.26 92.71) (width 0.25) (layer F.Cu) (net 21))
 (segment (start 153.67 88.9) (end 157.48 92.71) (width 0.25) (layer F.Cu) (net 21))
 (segment (start 153.67 83.82) (end 153.67 88.9) (width 0.25) (layer F.Cu) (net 21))
 (segment (start 153.67 83.82) (end 153.67 83.82) (width 0.25) (layer F.Cu) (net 21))
 (segment (start 146.685 83.82) (end 153.67 83.82) (width 0.25) (layer F.Cu) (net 21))
 (segment (start 146.05 84.455) (end 146.685 83.82) (width 0.25) (layer F.Cu) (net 21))
 (segment (start 146.05 86.995) (end 146.05 84.455) (width 0.25) (layer F.Cu) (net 21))
 (segment (start 190.5 120.65) (end 189.23 121.92) (width 0.25) (layer F.Cu) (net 33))
 (segment (start 189.23 121.92) (end 166.37 121.92) (width 0.25) (layer F.Cu) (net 33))
 (segment (start 189.23 119.38) (end 190.5 120.65) (width 0.25) (layer F.Cu) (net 33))
 (segment (start 185.42 119.38) (end 189.23 119.38) (width 0.25) (layer F.Cu) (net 33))
 (segment (start 179.07 113.03) (end 185.42 119.38) (width 0.25) (layer F.Cu) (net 33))
 (segment (start 161.29 113.03) (end 179.07 113.03) (width 0.25) (layer F.Cu) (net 33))
 (segment (start 160.02 114.3) (end 161.29 113.03) (width 0.25) (layer F.Cu) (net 33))
 (segment (start 160.02 116.84) (end 160.02 114.3) (width 0.25) (layer F.Cu) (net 33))
 (segment (start 158.75 118.11) (end 160.02 116.84) (width 0.25) (layer F.Cu) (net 33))
 (segment (start 147.955 118.11) (end 158.75 118.11) (width 0.25) (layer F.Cu) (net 33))
 (segment (start 146.685 116.84) (end 147.955 118.11) (width 0.25) (layer F.Cu) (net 33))
 (segment (start 146.685 92.71) (end 146.685 116.84) (width 0.25) (layer F.Cu) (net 33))
 (segment (start 143.35 85.725) (end 144.78 85.725) (width 0.25) (layer F.Cu) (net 41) (status 400000))
 (segment (start 189.23 101.6) (end 190.5 102.87) (width 0.25) (layer F.Cu) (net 41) (status 800000))
 (segment (start 186.69 101.6) (end 189.23 101.6) (width 0.25) (layer F.Cu) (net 41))
 (segment (start 177.165 92.075) (end 186.69 101.6) (width 0.25) (layer F.Cu) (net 41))
 (segment (start 157.48 92.075) (end 177.165 92.075) (width 0.25) (layer F.Cu) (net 41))
 (segment (start 154.305 88.9) (end 157.48 92.075) (width 0.25) (layer F.Cu) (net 41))
 (segment (start 154.305 83.82) (end 154.305 88.9) (width 0.25) (layer F.Cu) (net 41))
 (segment (start 153.67 83.185) (end 154.305 83.82) (width 0.25) (layer F.Cu) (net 41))
 (segment (start 146.05 83.185) (end 153.67 83.185) (width 0.25) (layer F.Cu) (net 41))
 (segment (start 145.415 83.82) (end 146.05 83.185) (width 0.25) (layer F.Cu) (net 41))
 (segment (start 145.415 85.09) (end 145.415 83.82) (width 0.25) (layer F.Cu) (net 41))
 (segment (start 144.78 85.725) (end 145.415 85.09) (width 0.25) (layer F.Cu) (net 41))
 (segment (start 165.1 85.09) (end 165.1 81.28) (width 0.25) (layer F.Cu) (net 41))
 (segment (start 157.48 113.03) (end 157.48 115.57) (width 0.25) (layer F.Cu) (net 41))
 (segment (start 158.75 111.76) (end 157.48 113.03) (width 0.25) (layer F.Cu) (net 41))
 (segment (start 157.48 108.585) (end 157.48 104.14) (width 0.25) (layer F.Cu) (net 41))
 (segment (start 158.75 109.855) (end 157.48 108.585) (width 0.25) (layer F.Cu) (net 41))
 (segment (start 186.055 109.855) (end 158.75 109.855) (width 0.25) (layer F.Cu) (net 41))
 (segment (start 166.37 121.92) (end 166.37 127) (width 0.25) (layer F.Cu) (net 41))
 (segment (start 143.35 92.075) (end 146.05 92.075) (width 0.25) (layer F.Cu) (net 41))
 (segment (start 146.05 92.075) (end 146.685 92.71) (width 0.25) (layer F.Cu) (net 41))
 (segment (start 179.07 104.14) (end 179.07 108.585) (width 0.25) (layer F.Cu) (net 41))
 (segment (start 179.07 108.585) (end 179.705 109.22) (width 0.25) (layer F.Cu) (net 41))
 (segment (start 148.75 94.615) (end 150.495 94.615) (width 0.25) (layer F.Cu) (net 43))
 (segment (start 152.4 112.395) (end 152.4 115.57) (width 0.25) (layer F.Cu) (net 43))
 (segment (start 151.13 111.125) (end 152.4 112.395) (width 0.25) (layer F.Cu) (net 43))
 (segment (start 151.13 95.25) (end 151.13 111.125) (width 0.25) (layer F.Cu) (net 43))
 (segment (start 150.495 94.615) (end 151.13 95.25) (width 0.25) (layer F.Cu) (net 43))
 (segment (start 149.225 93.345) (end 148.75 93.345) (width 0.25) (layer F.Cu) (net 44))
 (segment (start 148.75 93.345) (end 151.765 93.345) (width 0.25) (layer F.Cu) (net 44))
 (segment (start 152.4 93.98) (end 152.4 104.14) (width 0.25) (layer F.Cu) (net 44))
 (segment (start 151.765 93.345) (end 152.4 93.98) (width 0.25) (layer F.Cu) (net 44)))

